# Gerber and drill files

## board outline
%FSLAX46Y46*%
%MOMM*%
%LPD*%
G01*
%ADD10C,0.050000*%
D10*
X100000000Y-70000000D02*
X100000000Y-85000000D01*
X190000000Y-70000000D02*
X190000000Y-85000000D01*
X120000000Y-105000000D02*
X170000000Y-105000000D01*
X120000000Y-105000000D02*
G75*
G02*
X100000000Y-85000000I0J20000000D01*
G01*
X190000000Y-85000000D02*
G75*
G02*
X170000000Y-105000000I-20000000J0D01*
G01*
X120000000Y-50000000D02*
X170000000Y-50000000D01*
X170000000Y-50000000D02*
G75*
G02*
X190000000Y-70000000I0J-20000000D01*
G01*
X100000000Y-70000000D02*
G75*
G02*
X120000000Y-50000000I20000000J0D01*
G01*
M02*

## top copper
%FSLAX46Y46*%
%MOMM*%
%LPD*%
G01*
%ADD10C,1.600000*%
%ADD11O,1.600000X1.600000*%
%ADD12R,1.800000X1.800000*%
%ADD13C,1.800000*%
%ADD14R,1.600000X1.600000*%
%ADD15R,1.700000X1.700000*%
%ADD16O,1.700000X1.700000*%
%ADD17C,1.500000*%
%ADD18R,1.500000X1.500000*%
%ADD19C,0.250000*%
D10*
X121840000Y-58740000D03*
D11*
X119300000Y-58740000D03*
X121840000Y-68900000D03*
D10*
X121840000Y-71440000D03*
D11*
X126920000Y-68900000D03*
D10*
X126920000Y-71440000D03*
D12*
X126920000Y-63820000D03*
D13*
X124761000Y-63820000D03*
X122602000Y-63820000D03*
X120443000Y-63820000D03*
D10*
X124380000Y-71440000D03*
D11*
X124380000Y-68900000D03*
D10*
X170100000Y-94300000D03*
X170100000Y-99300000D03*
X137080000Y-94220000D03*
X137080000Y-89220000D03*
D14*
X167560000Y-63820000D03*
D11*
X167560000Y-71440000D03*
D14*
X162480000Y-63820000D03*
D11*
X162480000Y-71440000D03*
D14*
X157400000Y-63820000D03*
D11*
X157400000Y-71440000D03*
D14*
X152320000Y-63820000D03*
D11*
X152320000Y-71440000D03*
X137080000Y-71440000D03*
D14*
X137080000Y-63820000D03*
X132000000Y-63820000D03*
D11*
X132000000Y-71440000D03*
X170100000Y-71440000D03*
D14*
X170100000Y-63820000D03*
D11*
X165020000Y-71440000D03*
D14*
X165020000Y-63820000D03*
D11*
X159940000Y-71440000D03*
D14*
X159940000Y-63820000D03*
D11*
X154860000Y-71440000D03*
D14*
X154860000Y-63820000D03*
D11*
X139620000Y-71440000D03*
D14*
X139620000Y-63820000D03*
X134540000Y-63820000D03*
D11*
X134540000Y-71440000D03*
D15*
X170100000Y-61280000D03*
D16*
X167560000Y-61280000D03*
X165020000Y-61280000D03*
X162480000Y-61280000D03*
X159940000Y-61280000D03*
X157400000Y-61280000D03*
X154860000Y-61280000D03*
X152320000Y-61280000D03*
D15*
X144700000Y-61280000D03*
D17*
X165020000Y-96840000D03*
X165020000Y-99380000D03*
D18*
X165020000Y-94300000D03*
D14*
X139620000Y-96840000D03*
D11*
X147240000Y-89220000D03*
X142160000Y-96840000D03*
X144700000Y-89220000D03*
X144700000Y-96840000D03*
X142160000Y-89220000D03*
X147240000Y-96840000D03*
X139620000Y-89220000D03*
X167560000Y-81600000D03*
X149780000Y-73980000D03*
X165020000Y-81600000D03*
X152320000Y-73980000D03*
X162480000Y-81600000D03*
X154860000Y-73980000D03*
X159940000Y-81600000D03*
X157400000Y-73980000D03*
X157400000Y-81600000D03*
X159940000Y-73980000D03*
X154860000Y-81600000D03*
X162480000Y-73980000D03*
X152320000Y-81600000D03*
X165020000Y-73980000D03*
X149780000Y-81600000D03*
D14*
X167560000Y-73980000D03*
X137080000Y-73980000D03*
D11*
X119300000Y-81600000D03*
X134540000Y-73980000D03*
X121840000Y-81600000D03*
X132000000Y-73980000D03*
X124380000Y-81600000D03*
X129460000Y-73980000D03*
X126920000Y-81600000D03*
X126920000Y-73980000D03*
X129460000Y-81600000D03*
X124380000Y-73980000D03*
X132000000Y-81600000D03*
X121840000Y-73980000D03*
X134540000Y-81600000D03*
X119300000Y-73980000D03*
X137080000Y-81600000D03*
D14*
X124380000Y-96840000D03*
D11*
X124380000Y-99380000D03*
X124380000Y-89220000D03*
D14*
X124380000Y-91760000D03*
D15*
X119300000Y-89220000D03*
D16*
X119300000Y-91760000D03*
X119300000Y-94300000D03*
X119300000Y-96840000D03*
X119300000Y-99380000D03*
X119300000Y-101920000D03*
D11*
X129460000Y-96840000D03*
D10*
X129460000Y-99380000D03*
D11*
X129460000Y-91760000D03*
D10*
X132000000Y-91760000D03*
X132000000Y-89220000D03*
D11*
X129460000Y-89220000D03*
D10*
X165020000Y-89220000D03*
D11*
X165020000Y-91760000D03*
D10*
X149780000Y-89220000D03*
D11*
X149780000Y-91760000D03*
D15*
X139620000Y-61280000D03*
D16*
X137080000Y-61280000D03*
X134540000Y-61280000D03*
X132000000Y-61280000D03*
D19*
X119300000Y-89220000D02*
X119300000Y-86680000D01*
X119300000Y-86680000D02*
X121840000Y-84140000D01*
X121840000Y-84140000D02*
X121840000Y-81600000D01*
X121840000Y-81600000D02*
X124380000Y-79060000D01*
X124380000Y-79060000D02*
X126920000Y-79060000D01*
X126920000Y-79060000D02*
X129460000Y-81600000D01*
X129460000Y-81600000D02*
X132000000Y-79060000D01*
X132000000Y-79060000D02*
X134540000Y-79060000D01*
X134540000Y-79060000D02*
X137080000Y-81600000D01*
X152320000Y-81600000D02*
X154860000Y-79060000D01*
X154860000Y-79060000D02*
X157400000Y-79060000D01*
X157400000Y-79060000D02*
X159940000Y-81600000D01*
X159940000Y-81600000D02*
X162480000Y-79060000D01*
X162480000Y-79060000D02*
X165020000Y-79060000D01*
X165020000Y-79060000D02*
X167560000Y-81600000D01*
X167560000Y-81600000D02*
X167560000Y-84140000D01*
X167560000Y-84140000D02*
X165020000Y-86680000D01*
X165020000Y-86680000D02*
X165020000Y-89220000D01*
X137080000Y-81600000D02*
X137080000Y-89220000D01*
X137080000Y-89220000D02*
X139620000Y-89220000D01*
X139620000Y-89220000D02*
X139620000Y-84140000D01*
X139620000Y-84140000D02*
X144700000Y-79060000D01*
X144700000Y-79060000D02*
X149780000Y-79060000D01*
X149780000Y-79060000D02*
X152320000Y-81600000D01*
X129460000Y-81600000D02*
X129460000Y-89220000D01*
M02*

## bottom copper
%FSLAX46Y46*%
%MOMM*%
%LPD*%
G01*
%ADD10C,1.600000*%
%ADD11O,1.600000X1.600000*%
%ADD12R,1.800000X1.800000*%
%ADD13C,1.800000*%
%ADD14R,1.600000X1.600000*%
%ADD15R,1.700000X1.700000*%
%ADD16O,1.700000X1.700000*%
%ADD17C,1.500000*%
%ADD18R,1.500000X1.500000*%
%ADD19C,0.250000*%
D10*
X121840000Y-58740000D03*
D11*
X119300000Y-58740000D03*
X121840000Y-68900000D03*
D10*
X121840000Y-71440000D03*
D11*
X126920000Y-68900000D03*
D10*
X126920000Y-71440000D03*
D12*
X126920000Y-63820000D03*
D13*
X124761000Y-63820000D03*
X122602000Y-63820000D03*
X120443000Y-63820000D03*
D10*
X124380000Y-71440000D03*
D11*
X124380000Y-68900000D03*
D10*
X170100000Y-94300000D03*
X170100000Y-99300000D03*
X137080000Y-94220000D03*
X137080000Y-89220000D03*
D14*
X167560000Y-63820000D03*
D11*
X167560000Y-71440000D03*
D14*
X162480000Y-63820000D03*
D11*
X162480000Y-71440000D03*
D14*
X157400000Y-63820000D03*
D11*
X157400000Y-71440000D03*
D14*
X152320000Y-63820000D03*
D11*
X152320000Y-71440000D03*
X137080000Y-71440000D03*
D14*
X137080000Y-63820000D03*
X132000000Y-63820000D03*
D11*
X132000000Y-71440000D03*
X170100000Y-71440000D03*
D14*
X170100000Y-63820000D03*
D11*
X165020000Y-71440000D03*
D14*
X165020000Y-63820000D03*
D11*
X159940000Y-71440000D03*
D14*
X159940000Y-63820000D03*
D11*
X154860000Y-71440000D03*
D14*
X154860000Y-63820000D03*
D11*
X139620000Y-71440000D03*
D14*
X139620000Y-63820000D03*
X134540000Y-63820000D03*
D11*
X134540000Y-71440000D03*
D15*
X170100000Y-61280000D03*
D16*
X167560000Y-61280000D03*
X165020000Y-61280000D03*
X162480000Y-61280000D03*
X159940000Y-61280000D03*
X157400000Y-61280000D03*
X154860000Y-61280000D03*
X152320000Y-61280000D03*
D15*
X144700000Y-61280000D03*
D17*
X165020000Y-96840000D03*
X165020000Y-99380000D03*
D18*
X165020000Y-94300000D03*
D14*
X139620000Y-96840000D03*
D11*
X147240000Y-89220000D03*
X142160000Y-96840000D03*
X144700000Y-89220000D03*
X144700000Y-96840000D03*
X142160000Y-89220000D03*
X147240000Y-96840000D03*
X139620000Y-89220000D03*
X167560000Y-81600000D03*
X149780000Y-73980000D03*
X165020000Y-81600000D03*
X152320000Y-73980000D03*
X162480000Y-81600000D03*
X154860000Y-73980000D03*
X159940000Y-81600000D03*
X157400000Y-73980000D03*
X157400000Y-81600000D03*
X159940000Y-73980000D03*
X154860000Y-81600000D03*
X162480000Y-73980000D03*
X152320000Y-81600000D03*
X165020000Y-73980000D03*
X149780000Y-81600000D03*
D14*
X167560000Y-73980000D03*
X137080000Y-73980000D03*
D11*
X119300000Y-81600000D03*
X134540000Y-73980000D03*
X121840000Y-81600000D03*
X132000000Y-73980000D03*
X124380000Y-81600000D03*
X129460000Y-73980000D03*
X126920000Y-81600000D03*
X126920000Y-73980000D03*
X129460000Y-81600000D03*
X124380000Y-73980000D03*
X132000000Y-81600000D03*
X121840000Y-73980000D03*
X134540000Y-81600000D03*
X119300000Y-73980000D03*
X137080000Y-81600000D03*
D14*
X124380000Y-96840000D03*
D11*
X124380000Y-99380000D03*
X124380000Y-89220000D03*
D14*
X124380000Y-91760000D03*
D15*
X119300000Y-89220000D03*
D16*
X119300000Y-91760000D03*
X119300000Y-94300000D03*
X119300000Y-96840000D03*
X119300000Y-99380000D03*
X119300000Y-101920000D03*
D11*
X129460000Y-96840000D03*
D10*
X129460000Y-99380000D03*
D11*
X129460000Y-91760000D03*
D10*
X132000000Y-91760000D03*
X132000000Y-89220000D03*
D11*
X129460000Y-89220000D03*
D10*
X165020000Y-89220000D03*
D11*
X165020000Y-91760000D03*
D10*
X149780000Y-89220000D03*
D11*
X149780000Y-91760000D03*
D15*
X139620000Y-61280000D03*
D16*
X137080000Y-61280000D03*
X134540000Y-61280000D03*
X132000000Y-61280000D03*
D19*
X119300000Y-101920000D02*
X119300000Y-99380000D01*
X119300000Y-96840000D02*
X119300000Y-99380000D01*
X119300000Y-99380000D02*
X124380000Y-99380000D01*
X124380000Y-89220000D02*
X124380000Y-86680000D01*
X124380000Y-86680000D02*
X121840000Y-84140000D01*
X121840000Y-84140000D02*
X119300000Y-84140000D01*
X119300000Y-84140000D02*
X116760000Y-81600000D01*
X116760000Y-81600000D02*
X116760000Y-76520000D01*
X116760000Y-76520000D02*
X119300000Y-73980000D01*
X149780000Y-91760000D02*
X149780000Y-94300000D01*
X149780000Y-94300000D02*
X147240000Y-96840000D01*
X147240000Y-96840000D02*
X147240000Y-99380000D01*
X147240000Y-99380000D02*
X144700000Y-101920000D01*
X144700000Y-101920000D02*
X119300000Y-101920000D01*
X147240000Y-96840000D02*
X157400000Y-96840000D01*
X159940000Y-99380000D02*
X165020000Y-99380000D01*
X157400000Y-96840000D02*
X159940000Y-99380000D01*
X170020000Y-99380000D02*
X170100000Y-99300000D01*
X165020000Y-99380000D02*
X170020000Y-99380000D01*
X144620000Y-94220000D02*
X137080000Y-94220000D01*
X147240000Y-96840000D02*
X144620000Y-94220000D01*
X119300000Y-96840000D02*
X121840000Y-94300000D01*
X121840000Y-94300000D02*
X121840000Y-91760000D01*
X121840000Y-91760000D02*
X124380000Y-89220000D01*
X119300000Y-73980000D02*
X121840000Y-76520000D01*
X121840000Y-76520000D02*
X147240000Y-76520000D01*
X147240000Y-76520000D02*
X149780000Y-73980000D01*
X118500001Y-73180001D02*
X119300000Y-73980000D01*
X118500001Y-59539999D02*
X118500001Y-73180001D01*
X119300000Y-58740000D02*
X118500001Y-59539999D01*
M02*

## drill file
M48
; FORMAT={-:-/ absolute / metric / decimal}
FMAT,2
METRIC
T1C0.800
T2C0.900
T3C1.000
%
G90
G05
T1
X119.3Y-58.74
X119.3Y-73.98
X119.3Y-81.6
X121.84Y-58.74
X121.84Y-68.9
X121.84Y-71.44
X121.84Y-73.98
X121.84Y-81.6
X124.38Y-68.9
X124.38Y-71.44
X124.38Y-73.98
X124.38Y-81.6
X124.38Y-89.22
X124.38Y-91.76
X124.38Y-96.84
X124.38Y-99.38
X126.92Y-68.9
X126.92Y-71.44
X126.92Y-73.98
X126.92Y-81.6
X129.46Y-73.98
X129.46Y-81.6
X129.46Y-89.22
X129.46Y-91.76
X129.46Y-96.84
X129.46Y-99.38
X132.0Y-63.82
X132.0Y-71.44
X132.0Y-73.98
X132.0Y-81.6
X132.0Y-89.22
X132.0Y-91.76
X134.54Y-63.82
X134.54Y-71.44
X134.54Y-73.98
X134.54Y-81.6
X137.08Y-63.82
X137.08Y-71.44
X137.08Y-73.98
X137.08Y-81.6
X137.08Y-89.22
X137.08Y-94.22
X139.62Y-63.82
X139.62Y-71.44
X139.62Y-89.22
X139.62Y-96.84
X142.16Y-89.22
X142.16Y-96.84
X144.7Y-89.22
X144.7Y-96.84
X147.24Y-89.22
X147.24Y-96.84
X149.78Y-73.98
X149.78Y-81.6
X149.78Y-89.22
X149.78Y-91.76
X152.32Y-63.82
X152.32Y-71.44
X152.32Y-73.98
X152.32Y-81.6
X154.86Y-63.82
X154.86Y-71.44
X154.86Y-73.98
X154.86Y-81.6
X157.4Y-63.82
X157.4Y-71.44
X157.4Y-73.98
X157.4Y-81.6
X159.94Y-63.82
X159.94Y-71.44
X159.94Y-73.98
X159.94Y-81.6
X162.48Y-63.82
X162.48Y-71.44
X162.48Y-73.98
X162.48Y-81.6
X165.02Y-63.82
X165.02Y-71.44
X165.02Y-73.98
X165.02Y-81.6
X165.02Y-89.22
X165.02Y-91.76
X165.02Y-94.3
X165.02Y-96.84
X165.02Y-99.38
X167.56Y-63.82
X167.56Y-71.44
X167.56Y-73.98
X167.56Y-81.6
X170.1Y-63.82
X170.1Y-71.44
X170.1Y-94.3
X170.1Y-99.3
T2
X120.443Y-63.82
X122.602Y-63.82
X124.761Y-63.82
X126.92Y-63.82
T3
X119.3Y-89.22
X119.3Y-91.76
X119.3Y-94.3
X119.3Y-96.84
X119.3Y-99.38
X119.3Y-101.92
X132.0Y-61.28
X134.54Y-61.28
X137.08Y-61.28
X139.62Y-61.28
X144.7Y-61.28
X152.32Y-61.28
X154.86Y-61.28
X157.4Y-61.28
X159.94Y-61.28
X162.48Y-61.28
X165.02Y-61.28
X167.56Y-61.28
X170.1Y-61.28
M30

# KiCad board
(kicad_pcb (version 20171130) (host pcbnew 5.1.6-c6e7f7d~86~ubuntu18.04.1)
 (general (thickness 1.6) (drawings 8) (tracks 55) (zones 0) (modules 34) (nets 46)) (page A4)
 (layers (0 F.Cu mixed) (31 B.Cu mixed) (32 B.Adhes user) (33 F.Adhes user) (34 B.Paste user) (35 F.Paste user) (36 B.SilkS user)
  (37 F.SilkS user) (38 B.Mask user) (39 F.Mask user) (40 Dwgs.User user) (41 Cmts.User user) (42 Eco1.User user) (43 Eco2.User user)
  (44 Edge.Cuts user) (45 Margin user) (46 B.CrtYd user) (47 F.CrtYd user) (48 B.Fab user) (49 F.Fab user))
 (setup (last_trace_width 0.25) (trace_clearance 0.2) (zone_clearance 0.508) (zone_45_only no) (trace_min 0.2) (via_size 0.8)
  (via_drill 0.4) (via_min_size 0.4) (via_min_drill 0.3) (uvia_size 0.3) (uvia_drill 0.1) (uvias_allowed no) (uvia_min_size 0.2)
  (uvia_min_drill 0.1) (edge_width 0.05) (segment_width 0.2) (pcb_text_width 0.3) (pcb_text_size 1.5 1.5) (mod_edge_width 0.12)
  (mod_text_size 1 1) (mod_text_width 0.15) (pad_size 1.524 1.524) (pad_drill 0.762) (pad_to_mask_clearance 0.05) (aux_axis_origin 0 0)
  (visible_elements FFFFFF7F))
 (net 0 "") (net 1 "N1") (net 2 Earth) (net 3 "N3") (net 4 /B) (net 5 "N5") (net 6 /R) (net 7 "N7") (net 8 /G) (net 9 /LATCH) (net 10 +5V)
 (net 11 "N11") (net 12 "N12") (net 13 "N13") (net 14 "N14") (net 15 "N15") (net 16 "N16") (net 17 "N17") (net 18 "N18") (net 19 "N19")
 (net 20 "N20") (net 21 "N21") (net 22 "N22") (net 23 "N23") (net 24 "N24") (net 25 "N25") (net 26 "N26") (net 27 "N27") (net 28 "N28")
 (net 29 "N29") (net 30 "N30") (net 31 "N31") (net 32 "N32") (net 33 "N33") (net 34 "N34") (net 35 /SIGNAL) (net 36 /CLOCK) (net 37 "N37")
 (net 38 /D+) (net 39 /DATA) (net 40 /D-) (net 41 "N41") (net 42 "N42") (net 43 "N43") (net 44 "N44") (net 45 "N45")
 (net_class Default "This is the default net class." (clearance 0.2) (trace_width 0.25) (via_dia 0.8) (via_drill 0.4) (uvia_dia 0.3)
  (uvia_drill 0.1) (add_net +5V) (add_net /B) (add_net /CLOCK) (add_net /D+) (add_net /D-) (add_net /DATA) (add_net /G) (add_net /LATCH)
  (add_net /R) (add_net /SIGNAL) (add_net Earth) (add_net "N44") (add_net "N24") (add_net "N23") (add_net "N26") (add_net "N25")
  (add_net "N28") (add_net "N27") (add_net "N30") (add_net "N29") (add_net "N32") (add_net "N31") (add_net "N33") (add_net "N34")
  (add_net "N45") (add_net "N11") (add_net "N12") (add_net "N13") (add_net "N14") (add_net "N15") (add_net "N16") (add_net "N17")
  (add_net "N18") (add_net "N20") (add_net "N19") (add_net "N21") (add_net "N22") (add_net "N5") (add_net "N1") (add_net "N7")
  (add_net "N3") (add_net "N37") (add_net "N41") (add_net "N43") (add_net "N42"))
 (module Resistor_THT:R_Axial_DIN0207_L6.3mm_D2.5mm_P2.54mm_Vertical (layer F.Cu) (at 121.84 58.74 180)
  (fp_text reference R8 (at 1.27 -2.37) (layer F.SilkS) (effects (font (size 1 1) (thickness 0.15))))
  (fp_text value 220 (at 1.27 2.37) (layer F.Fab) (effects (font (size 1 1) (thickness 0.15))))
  (pad 1 thru_hole circle (at 0 0 180) (size 1.6 1.6) (drill 0.8) (layers *.Cu *.Mask) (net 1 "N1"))
  (pad 2 thru_hole oval (at 2.54 0 180) (size 1.6 1.6) (drill 0.8) (layers *.Cu *.Mask) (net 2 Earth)))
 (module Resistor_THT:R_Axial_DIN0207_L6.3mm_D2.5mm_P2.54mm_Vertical (layer F.Cu) (at 121.84 71.44 90)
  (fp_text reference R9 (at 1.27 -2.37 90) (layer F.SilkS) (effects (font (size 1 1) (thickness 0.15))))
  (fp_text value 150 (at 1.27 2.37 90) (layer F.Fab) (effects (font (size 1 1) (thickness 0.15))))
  (pad 2 thru_hole oval (at 2.54 0 90) (size 1.6 1.6) (drill 0.8) (layers *.Cu *.Mask) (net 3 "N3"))
  (pad 1 thru_hole circle (at 0 0 90) (size 1.6 1.6) (drill 0.8) (layers *.Cu *.Mask) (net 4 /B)))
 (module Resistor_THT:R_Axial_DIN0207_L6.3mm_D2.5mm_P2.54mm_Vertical (layer F.Cu) (at 126.92 71.44 90)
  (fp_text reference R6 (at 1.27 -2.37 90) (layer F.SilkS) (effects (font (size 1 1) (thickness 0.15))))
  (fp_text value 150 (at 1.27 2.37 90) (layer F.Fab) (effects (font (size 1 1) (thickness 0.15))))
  (pad 2 thru_hole oval (at 2.54 0 90) (size 1.6 1.6) (drill 0.8) (layers *.Cu *.Mask) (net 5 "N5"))
  (pad 1 thru_hole circle (at 0 0 90) (size 1.6 1.6) (drill 0.8) (layers *.Cu *.Mask) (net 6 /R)))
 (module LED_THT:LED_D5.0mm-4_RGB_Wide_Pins (layer F.Cu) (at 126.92 63.82 180)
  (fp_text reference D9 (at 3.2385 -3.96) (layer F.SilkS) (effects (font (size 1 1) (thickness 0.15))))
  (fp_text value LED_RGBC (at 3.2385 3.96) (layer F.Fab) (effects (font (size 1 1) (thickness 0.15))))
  (pad 1 thru_hole rect (at 0 0 180) (size 1.8 1.8) (drill 0.9) (layers *.Cu *.Mask) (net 5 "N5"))
  (pad 2 thru_hole circle (at 2.159 0 180) (size 1.8 1.8) (drill 0.9) (layers *.Cu *.Mask) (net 1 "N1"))
  (pad 3 thru_hole circle (at 4.318 0 180) (size 1.8 1.8) (drill 0.9) (layers *.Cu *.Mask) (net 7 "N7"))
  (pad 4 thru_hole circle (at 6.477 0 180) (size 1.8 1.8) (drill 0.9) (layers *.Cu *.Mask) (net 3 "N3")))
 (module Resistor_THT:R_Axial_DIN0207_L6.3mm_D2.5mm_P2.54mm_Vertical (layer F.Cu) (at 124.38 71.44 90)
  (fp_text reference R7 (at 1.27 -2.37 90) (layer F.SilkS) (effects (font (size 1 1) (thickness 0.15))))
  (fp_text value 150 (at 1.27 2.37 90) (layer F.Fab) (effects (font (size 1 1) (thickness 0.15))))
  (pad 1 thru_hole circle (at 0 0 90) (size 1.6 1.6) (drill 0.8) (layers *.Cu *.Mask) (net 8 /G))
  (pad 2 thru_hole oval (at 2.54 0 90) (size 1.6 1.6) (drill 0.8) (layers *.Cu *.Mask) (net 7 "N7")))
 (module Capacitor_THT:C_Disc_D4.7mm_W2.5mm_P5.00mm (layer F.Cu) (at 170.1 94.3 270)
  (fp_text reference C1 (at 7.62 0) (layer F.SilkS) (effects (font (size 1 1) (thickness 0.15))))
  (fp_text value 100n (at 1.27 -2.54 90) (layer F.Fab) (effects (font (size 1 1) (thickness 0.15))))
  (pad 1 thru_hole circle (at 0 0 270) (size 1.6 1.6) (drill 0.8) (layers *.Cu *.Mask) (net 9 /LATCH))
  (pad 2 thru_hole circle (at 5 0 270) (size 1.6 1.6) (drill 0.8) (layers *.Cu *.Mask) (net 2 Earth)))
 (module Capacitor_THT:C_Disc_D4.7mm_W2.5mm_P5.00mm (layer F.Cu) (at 137.08 89.22 270)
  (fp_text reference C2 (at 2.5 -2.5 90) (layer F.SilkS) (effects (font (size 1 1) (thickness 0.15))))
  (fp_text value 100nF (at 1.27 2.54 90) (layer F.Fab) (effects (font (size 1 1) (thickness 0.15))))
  (pad 2 thru_hole circle (at 5 0 270) (size 1.6 1.6) (drill 0.8) (layers *.Cu *.Mask) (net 2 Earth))
  (pad 1 thru_hole circle (at 0 0 270) (size 1.6 1.6) (drill 0.8) (layers *.Cu *.Mask) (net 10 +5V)))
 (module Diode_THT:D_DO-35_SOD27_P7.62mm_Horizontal (layer F.Cu) (at 167.56 63.82 270)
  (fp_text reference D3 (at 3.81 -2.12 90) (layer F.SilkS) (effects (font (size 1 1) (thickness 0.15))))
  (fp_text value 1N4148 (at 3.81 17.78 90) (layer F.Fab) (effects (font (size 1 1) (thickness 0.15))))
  (pad 1 thru_hole rect (at 0 0 270) (size 1.6 1.6) (drill 0.8) (layers *.Cu *.Mask) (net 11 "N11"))
  (pad 2 thru_hole oval (at 7.62 0 270) (size 1.6 1.6) (drill 0.8) (layers *.Cu *.Mask) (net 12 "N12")))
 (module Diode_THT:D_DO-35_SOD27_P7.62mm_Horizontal (layer F.Cu) (at 162.48 63.82 270)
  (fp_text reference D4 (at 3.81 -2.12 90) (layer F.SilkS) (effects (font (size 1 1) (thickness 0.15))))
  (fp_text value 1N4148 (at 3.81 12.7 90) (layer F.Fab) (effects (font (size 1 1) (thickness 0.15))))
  (pad 1 thru_hole rect (at 0 0 270) (size 1.6 1.6) (drill 0.8) (layers *.Cu *.Mask) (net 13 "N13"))
  (pad 2 thru_hole oval (at 7.62 0 270) (size 1.6 1.6) (drill 0.8) (layers *.Cu *.Mask) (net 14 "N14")))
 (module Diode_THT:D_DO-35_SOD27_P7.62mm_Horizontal (layer F.Cu) (at 157.4 63.82 270)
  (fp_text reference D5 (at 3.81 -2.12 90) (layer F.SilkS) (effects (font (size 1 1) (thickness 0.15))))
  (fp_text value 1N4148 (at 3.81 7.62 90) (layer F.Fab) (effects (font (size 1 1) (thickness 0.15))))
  (pad 1 thru_hole rect (at 0 0 270) (size 1.6 1.6) (drill 0.8) (layers *.Cu *.Mask) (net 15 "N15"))
  (pad 2 thru_hole oval (at 7.62 0 270) (size 1.6 1.6) (drill 0.8) (layers *.Cu *.Mask) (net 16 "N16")))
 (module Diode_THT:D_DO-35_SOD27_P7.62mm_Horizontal (layer F.Cu) (at 152.32 63.82 270)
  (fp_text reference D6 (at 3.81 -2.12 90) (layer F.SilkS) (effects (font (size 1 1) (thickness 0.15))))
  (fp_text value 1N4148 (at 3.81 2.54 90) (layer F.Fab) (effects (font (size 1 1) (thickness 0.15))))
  (pad 1 thru_hole rect (at 0 0 270) (size 1.6 1.6) (drill 0.8) (layers *.Cu *.Mask) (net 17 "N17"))
  (pad 2 thru_hole oval (at 7.62 0 270) (size 1.6 1.6) (drill 0.8) (layers *.Cu *.Mask) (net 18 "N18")))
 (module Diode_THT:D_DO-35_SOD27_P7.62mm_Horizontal (layer F.Cu) (at 137.08 63.82 270)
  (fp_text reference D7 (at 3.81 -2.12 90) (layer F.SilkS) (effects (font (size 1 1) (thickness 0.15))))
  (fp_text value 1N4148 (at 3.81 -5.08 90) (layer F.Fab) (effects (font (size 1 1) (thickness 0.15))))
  (pad 2 thru_hole oval (at 7.62 0 270) (size 1.6 1.6) (drill 0.8) (layers *.Cu *.Mask) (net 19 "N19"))
  (pad 1 thru_hole rect (at 0 0 270) (size 1.6 1.6) (drill 0.8) (layers *.Cu *.Mask) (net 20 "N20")))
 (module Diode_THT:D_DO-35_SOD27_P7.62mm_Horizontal (layer F.Cu) (at 132 63.82 270)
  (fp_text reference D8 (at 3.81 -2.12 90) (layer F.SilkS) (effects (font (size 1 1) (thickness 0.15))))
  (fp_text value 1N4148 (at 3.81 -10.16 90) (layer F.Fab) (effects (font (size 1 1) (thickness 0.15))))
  (pad 1 thru_hole rect (at 0 0 270) (size 1.6 1.6) (drill 0.8) (layers *.Cu *.Mask) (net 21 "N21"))
  (pad 2 thru_hole oval (at 7.62 0 270) (size 1.6 1.6) (drill 0.8) (layers *.Cu *.Mask) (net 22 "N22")))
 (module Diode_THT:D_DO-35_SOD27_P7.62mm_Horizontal (layer F.Cu) (at 170.1 63.82 270)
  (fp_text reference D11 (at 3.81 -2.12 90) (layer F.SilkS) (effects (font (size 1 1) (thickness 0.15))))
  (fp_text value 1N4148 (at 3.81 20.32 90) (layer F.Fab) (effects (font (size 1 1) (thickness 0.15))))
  (pad 2 thru_hole oval (at 7.62 0 270) (size 1.6 1.6) (drill 0.8) (layers *.Cu *.Mask) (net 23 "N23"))
  (pad 1 thru_hole rect (at 0 0 270) (size 1.6 1.6) (drill 0.8) (layers *.Cu *.Mask) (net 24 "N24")))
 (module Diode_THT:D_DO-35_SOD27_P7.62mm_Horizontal (layer F.Cu) (at 165.02 63.82 270)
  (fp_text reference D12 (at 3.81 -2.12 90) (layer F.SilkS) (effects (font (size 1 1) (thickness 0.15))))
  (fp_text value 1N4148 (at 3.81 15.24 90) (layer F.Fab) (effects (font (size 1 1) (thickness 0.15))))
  (pad 2 thru_hole oval (at 7.62 0 270) (size 1.6 1.6) (drill 0.8) (layers *.Cu *.Mask) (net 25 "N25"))
  (pad 1 thru_hole rect (at 0 0 270) (size 1.6 1.6) (drill 0.8) (layers *.Cu *.Mask) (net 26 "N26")))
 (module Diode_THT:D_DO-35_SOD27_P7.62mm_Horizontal (layer F.Cu) (at 159.94 63.82 270)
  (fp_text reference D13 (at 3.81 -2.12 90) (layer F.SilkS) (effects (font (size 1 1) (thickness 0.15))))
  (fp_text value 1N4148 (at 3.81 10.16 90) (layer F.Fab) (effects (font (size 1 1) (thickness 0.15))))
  (pad 2 thru_hole oval (at 7.62 0 270) (size 1.6 1.6) (drill 0.8) (layers *.Cu *.Mask) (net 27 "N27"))
  (pad 1 thru_hole rect (at 0 0 270) (size 1.6 1.6) (drill 0.8) (layers *.Cu *.Mask) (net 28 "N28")))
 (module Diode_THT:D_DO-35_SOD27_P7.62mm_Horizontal (layer F.Cu) (at 154.86 63.82 270)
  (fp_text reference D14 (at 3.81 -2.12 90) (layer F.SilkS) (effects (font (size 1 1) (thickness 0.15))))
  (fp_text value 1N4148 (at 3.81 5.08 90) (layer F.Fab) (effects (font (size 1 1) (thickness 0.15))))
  (pad 2 thru_hole oval (at 7.62 0 270) (size 1.6 1.6) (drill 0.8) (layers *.Cu *.Mask) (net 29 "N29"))
  (pad 1 thru_hole rect (at 0 0 270) (size 1.6 1.6) (drill 0.8) (layers *.Cu *.Mask) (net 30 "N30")))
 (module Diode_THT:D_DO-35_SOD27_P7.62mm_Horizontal (layer F.Cu) (at 139.62 63.82 270)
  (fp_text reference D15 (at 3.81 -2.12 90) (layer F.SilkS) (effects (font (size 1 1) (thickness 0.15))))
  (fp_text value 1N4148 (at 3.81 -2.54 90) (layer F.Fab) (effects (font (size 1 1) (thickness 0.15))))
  (pad 2 thru_hole oval (at 7.62 0 270) (size 1.6 1.6) (drill 0.8) (layers *.Cu *.Mask) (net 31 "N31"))
  (pad 1 thru_hole rect (at 0 0 270) (size 1.6 1.6) (drill 0.8) (layers *.Cu *.Mask) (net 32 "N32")))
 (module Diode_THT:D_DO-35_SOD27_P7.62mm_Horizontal (layer F.Cu) (at 134.54 63.82 270)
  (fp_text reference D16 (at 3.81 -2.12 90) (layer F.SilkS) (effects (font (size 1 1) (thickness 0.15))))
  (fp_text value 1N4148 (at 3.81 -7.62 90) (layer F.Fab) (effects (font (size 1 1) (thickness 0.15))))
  (pad 1 thru_hole rect (at 0 0 270) (size 1.6 1.6) (drill 0.8) (layers *.Cu *.Mask) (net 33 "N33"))
  (pad 2 thru_hole oval (at 7.62 0 270) (size 1.6 1.6) (drill 0.8) (layers *.Cu *.Mask) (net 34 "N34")))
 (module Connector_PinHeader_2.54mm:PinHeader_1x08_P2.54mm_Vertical (layer F.Cu) (at 170.1 61.28 270)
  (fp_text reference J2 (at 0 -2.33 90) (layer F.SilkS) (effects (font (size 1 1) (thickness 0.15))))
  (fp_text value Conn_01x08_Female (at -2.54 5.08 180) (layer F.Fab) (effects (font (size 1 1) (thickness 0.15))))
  (pad 1 thru_hole rect (at 0 0 270) (size 1.7 1.7) (drill 1) (layers *.Cu *.Mask) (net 24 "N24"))
  (pad 2 thru_hole oval (at 0 2.54 270) (size 1.7 1.7) (drill 1) (layers *.Cu *.Mask) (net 11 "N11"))
  (pad 3 thru_hole oval (at 0 5.08 270) (size 1.7 1.7) (drill 1) (layers *.Cu *.Mask) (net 26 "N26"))
  (pad 4 thru_hole oval (at 0 7.62 270) (size 1.7 1.7) (drill 1) (layers *.Cu *.Mask) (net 13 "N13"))
  (pad 5 thru_hole oval (at 0 10.16 270) (size 1.7 1.7) (drill 1) (layers *.Cu *.Mask) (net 28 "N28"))
  (pad 6 thru_hole oval (at 0 12.7 270) (size 1.7 1.7) (drill 1) (layers *.Cu *.Mask) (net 15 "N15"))
  (pad 7 thru_hole oval (at 0 15.24 270) (size 1.7 1.7) (drill 1) (layers *.Cu *.Mask) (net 30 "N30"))
  (pad 8 thru_hole oval (at 0 17.78 270) (size 1.7 1.7) (drill 1) (layers *.Cu *.Mask) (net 17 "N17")))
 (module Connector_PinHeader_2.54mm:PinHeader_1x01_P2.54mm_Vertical (layer F.Cu) (at 144.7 61.28)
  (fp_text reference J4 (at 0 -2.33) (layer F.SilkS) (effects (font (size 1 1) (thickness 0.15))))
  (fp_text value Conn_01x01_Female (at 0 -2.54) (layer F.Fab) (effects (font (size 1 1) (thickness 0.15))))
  (pad 1 thru_hole rect (at 0 0) (size 1.7 1.7) (drill 1) (layers *.Cu *.Mask) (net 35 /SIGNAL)))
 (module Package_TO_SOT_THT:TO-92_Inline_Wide (layer F.Cu) (at 165.02 94.3 270)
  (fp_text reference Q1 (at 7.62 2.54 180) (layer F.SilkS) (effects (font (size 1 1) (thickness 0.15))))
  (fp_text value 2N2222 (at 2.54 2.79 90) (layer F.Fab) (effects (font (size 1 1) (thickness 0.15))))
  (pad 2 thru_hole circle (at 2.54 0) (size 1.5 1.5) (drill 0.8) (layers *.Cu *.Mask) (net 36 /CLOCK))
  (pad 3 thru_hole circle (at 5.08 0) (size 1.5 1.5) (drill 0.8) (layers *.Cu *.Mask) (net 2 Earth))
  (pad 1 thru_hole rect (at 0 0) (size 1.5 1.5) (drill 0.8) (layers *.Cu *.Mask) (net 9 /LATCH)))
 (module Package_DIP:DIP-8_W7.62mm (layer F.Cu) (at 139.62 96.84 90)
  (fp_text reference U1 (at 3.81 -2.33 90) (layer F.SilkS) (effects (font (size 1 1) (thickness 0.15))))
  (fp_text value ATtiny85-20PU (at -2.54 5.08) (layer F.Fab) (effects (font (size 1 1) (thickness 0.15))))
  (pad 1 thru_hole rect (at 0 0 90) (size 1.6 1.6) (drill 0.8) (layers *.Cu *.Mask) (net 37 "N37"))
  (pad 5 thru_hole oval (at 7.62 7.62 90) (size 1.6 1.6) (drill 0.8) (layers *.Cu *.Mask) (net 35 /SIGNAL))
  (pad 2 thru_hole oval (at 0 2.54 90) (size 1.6 1.6) (drill 0.8) (layers *.Cu *.Mask) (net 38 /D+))
  (pad 6 thru_hole oval (at 7.62 5.08 90) (size 1.6 1.6) (drill 0.8) (layers *.Cu *.Mask) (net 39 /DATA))
  (pad 3 thru_hole oval (at 0 5.08 90) (size 1.6 1.6) (drill 0.8) (layers *.Cu *.Mask) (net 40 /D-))
  (pad 7 thru_hole oval (at 7.62 2.54 90) (size 1.6 1.6) (drill 0.8) (layers *.Cu *.Mask) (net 36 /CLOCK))
  (pad 4 thru_hole oval (at 0 7.62 90) (size 1.6 1.6) (drill 0.8) (layers *.Cu *.Mask) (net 2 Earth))
  (pad 8 thru_hole oval (at 7.62 0 90) (size 1.6 1.6) (drill 0.8) (layers *.Cu *.Mask) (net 10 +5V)))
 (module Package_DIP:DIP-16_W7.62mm (layer F.Cu) (at 167.56 73.98 270)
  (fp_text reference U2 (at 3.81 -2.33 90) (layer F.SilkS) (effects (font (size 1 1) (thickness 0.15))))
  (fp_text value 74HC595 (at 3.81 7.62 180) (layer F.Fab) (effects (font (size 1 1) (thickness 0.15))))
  (pad 16 thru_hole oval (at 7.62 0 270) (size 1.6 1.6) (drill 0.8) (layers *.Cu *.Mask) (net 10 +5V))
  (pad 8 thru_hole oval (at 0 17.78 270) (size 1.6 1.6) (drill 0.8) (layers *.Cu *.Mask) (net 2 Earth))
  (pad 15 thru_hole oval (at 7.62 2.54 270) (size 1.6 1.6) (drill 0.8) (layers *.Cu *.Mask) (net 23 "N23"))
  (pad 7 thru_hole oval (at 0 15.24 270) (size 1.6 1.6) (drill 0.8) (layers *.Cu *.Mask) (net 18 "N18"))
  (pad 14 thru_hole oval (at 7.62 5.08 270) (size 1.6 1.6) (drill 0.8) (layers *.Cu *.Mask) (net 39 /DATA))
  (pad 6 thru_hole oval (at 0 12.7 270) (size 1.6 1.6) (drill 0.8) (layers *.Cu *.Mask) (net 29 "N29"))
  (pad 13 thru_hole oval (at 7.62 7.62 270) (size 1.6 1.6) (drill 0.8) (layers *.Cu *.Mask) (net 10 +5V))
  (pad 5 thru_hole oval (at 0 10.16 270) (size 1.6 1.6) (drill 0.8) (layers *.Cu *.Mask) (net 16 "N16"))
  (pad 12 thru_hole oval (at 7.62 10.16 270) (size 1.6 1.6) (drill 0.8) (layers *.Cu *.Mask) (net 9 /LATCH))
  (pad 4 thru_hole oval (at 0 7.62 270) (size 1.6 1.6) (drill 0.8) (layers *.Cu *.Mask) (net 27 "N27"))
  (pad 11 thru_hole oval (at 7.62 12.7 270) (size 1.6 1.6) (drill 0.8) (layers *.Cu *.Mask) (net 36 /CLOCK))
  (pad 3 thru_hole oval (at 0 5.08 270) (size 1.6 1.6) (drill 0.8) (layers *.Cu *.Mask) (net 14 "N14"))
  (pad 10 thru_hole oval (at 7.62 15.24 270) (size 1.6 1.6) (drill 0.8) (layers *.Cu *.Mask) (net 10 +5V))
  (pad 2 thru_hole oval (at 0 2.54 270) (size 1.6 1.6) (drill 0.8) (layers *.Cu *.Mask) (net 25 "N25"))
  (pad 9 thru_hole oval (at 7.62 17.78 270) (size 1.6 1.6) (drill 0.8) (layers *.Cu *.Mask) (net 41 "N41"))
  (pad 1 thru_hole rect (at 0 0 270) (size 1.6 1.6) (drill 0.8) (layers *.Cu *.Mask) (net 12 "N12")))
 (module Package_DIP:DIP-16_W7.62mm (layer F.Cu) (at 137.08 73.98 270)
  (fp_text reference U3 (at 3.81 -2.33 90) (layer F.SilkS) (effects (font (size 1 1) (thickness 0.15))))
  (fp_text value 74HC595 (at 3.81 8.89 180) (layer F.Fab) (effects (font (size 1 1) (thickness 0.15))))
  (pad 1 thru_hole rect (at 0 0 270) (size 1.6 1.6) (drill 0.8) (layers *.Cu *.Mask) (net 19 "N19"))
  (pad 9 thru_hole oval (at 7.62 17.78 270) (size 1.6 1.6) (drill 0.8) (layers *.Cu *.Mask) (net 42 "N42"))
  (pad 2 thru_hole oval (at 0 2.54 270) (size 1.6 1.6) (drill 0.8) (layers *.Cu *.Mask) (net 34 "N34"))
  (pad 10 thru_hole oval (at 7.62 15.24 270) (size 1.6 1.6) (drill 0.8) (layers *.Cu *.Mask) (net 10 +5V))
  (pad 3 thru_hole oval (at 0 5.08 270) (size 1.6 1.6) (drill 0.8) (layers *.Cu *.Mask) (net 22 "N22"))
  (pad 11 thru_hole oval (at 7.62 12.7 270) (size 1.6 1.6) (drill 0.8) (layers *.Cu *.Mask) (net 36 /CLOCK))
  (pad 4 thru_hole oval (at 0 7.62 270) (size 1.6 1.6) (drill 0.8) (layers *.Cu *.Mask) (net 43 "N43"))
  (pad 12 thru_hole oval (at 7.62 10.16 270) (size 1.6 1.6) (drill 0.8) (layers *.Cu *.Mask) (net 9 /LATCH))
  (pad 5 thru_hole oval (at 0 10.16 270) (size 1.6 1.6) (drill 0.8) (layers *.Cu *.Mask) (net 6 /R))
  (pad 13 thru_hole oval (at 7.62 7.62 270) (size 1.6 1.6) (drill 0.8) (layers *.Cu *.Mask) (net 10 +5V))
  (pad 6 thru_hole oval (at 0 12.7 270) (size 1.6 1.6) (drill 0.8) (layers *.Cu *.Mask) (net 8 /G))
  (pad 14 thru_hole oval (at 7.62 5.08 270) (size 1.6 1.6) (drill 0.8) (layers *.Cu *.Mask) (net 41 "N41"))
  (pad 7 thru_hole oval (at 0 15.24 270) (size 1.6 1.6) (drill 0.8) (layers *.Cu *.Mask) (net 4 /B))
  (pad 15 thru_hole oval (at 7.62 2.54 270) (size 1.6 1.6) (drill 0.8) (layers *.Cu *.Mask) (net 31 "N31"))
  (pad 8 thru_hole oval (at 0 17.78 270) (size 1.6 1.6) (drill 0.8) (layers *.Cu *.Mask) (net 2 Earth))
  (pad 16 thru_hole oval (at 7.62 0 270) (size 1.6 1.6) (drill 0.8) (layers *.Cu *.Mask) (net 10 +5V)))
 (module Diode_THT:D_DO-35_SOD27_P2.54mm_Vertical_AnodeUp (layer F.Cu) (at 124.38 96.84 270)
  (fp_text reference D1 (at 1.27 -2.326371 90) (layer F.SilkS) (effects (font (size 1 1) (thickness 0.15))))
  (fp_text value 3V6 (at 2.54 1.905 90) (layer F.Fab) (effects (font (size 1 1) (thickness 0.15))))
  (pad 1 thru_hole rect (at 0 0 270) (size 1.6 1.6) (drill 0.8) (layers *.Cu *.Mask) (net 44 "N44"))
  (pad 2 thru_hole oval (at 2.54 0 270) (size 1.6 1.6) (drill 0.8) (layers *.Cu *.Mask) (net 2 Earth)))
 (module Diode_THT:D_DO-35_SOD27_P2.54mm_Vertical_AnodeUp (layer F.Cu) (at 124.38 91.76 90)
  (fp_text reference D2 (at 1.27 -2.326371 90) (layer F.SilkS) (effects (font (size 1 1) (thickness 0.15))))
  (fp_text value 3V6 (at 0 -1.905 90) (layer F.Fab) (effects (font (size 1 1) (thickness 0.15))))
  (pad 2 thru_hole oval (at 2.54 0 90) (size 1.6 1.6) (drill 0.8) (layers *.Cu *.Mask) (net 2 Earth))
  (pad 1 thru_hole rect (at 0 0 90) (size 1.6 1.6) (drill 0.8) (layers *.Cu *.Mask) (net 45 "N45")))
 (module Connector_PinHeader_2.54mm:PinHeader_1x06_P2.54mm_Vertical (layer F.Cu) (at 119.3 89.22)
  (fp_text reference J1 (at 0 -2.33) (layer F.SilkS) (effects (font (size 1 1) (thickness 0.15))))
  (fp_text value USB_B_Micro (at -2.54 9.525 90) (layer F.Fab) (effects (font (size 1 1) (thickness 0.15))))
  (pad 1 thru_hole rect (at 0 0) (size 1.7 1.7) (drill 1) (layers *.Cu *.Mask) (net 10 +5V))
  (pad 2 thru_hole oval (at 0 2.54) (size 1.7 1.7) (drill 1) (layers *.Cu *.Mask) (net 45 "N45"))
  (pad 3 thru_hole oval (at 0 5.08) (size 1.7 1.7) (drill 1) (layers *.Cu *.Mask) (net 44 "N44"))
  (pad 4 thru_hole oval (at 0 7.62) (size 1.7 1.7) (drill 1) (layers *.Cu *.Mask) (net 2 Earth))
  (pad 5 thru_hole oval (at 0 10.16) (size 1.7 1.7) (drill 1) (layers *.Cu *.Mask) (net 2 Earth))
  (pad 6 thru_hole oval (at 0 12.7) (size 1.7 1.7) (drill 1) (layers *.Cu *.Mask) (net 2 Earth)))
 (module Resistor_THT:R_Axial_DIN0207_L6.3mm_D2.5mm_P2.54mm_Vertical (layer F.Cu) (at 129.46 99.38 90)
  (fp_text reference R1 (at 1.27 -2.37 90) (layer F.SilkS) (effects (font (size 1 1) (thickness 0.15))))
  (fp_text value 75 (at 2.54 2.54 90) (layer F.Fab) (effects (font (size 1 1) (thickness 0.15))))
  (pad 2 thru_hole oval (at 2.54 0 90) (size 1.6 1.6) (drill 0.8) (layers *.Cu *.Mask) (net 44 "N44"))
  (pad 1 thru_hole circle (at 0 0 90) (size 1.6 1.6) (drill 0.8) (layers *.Cu *.Mask) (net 38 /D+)))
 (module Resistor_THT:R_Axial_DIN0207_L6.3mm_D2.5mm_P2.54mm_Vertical (layer F.Cu) (at 132 91.76 180)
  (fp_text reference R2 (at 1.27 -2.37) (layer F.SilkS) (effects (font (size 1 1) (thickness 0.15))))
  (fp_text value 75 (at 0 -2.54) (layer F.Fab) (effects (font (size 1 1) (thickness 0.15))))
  (pad 2 thru_hole oval (at 2.54 0 180) (size 1.6 1.6) (drill 0.8) (layers *.Cu *.Mask) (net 45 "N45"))
  (pad 1 thru_hole circle (at 0 0 180) (size 1.6 1.6) (drill 0.8) (layers *.Cu *.Mask) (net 40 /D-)))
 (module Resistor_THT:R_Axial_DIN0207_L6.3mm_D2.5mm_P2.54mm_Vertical (layer F.Cu) (at 132 89.22 180)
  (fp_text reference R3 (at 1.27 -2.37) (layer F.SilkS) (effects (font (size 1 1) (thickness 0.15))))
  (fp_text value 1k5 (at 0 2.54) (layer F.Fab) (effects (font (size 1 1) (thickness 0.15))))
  (pad 1 thru_hole circle (at 0 0 180) (size 1.6 1.6) (drill 0.8) (layers *.Cu *.Mask) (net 40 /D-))
  (pad 2 thru_hole oval (at 2.54 0 180) (size 1.6 1.6) (drill 0.8) (layers *.Cu *.Mask) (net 10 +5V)))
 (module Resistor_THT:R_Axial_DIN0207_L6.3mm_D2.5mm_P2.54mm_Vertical (layer F.Cu) (at 165.02 89.22 270)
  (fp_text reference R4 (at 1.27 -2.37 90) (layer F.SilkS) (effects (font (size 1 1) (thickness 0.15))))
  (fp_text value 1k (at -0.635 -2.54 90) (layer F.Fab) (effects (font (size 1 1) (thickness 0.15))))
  (pad 1 thru_hole circle (at 0 0 270) (size 1.6 1.6) (drill 0.8) (layers *.Cu *.Mask) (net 10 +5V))
  (pad 2 thru_hole oval (at 2.54 0 270) (size 1.6 1.6) (drill 0.8) (layers *.Cu *.Mask) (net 9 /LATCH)))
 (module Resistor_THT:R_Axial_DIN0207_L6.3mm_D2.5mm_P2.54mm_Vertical (layer F.Cu) (at 149.78 89.22 270)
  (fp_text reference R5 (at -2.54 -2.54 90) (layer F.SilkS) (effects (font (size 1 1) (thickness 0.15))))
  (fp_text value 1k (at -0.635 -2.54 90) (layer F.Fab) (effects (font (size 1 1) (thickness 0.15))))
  (pad 1 thru_hole circle (at 0 0 270) (size 1.6 1.6) (drill 0.8) (layers *.Cu *.Mask) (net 35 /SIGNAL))
  (pad 2 thru_hole oval (at 2.54 0 270) (size 1.6 1.6) (drill 0.8) (layers *.Cu *.Mask) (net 2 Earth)))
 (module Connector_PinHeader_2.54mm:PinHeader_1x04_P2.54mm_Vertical (layer F.Cu) (at 139.62 61.28 270)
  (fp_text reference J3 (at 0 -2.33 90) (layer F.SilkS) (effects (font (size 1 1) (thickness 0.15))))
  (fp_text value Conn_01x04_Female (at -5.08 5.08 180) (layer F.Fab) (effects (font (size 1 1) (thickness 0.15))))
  (pad 1 thru_hole rect (at 0 0 270) (size 1.7 1.7) (drill 1) (layers *.Cu *.Mask) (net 32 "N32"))
  (pad 2 thru_hole oval (at 0 2.54 270) (size 1.7 1.7) (drill 1) (layers *.Cu *.Mask) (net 20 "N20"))
  (pad 3 thru_hole oval (at 0 5.08 270) (size 1.7 1.7) (drill 1) (layers *.Cu *.Mask) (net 33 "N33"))
  (pad 4 thru_hole oval (at 0 7.62 270) (size 1.7 1.7) (drill 1) (layers *.Cu *.Mask) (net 21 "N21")))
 (gr_line (start 100 70) (end 100 85) (layer Edge.Cuts) (width 0.05))
 (gr_line (start 190 70) (end 190 85) (layer Edge.Cuts) (width 0.05))
 (gr_line (start 120 105) (end 170 105) (layer Edge.Cuts) (width 0.05))
 (gr_arc (start 120 85) (end 100 85) (angle -90) (layer Edge.Cuts) (width 0.05))
 (gr_arc (start 170 85) (end 170 105) (angle -90) (layer Edge.Cuts) (width 0.05))
 (gr_line (start 120 50) (end 170 50) (layer Edge.Cuts) (width 0.05))
 (gr_arc (start 170 70) (end 190 70) (angle -90) (layer Edge.Cuts) (width 0.05))
 (gr_arc (start 120 70) (end 120 50) (angle -90) (layer Edge.Cuts) (width 0.05))
 (segment (start 119.3 101.92) (end 119.3 99.38) (width 0.25) (layer B.Cu) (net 2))
 (segment (start 119.3 96.84) (end 119.3 99.38) (width 0.25) (layer B.Cu) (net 2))
 (segment (start 119.3 99.38) (end 124.38 99.38) (width 0.25) (layer B.Cu) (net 2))
 (segment (start 124.38 89.22) (end 124.38 86.68) (width 0.25) (layer B.Cu) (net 2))
 (segment (start 124.38 86.68) (end 121.84 84.14) (width 0.25) (layer B.Cu) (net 2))
 (segment (start 121.84 84.14) (end 119.3 84.14) (width 0.25) (layer B.Cu) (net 2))
 (segment (start 119.3 84.14) (end 116.76 81.6) (width 0.25) (layer B.Cu) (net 2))
 (segment (start 116.76 81.6) (end 116.76 76.52) (width 0.25) (layer B.Cu) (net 2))
 (segment (start 116.76 76.52) (end 119.3 73.98) (width 0.25) (layer B.Cu) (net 2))
 (segment (start 149.78 91.76) (end 149.78 94.3) (width 0.25) (layer B.Cu) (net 2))
 (segment (start 149.78 94.3) (end 147.24 96.84) (width 0.25) (layer B.Cu) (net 2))
 (segment (start 147.24 96.84) (end 147.24 99.38) (width 0.25) (layer B.Cu) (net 2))
 (segment (start 147.24 99.38) (end 144.7 101.92) (width 0.25) (layer B.Cu) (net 2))
 (segment (start 144.7 101.92) (end 119.3 101.92) (width 0.25) (layer B.Cu) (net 2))
 (segment (start 147.24 96.84) (end 157.4 96.84) (width 0.25) (layer B.Cu) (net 2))
 (segment (start 159.94 99.38) (end 165.02 99.38) (width 0.25) (layer B.Cu) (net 2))
 (segment (start 157.4 96.84) (end 159.94 99.38) (width 0.25) (layer B.Cu) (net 2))
 (segment (start 170.02 99.38) (end 170.1 99.3) (width 0.25) (layer B.Cu) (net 2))
 (segment (start 165.02 99.38) (end 170.02 99.38) (width 0.25) (layer B.Cu) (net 2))
 (segment (start 144.62 94.22) (end 137.08 94.22) (width 0.25) (layer B.Cu) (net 2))
 (segment (start 147.24 96.84) (end 144.62 94.22) (width 0.25) (layer B.Cu) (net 2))
 (segment (start 119.3 96.84) (end 121.84 94.3) (width 0.25) (layer B.Cu) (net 2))
 (segment (start 121.84 94.3) (end 121.84 91.76) (width 0.25) (layer B.Cu) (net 2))
 (segment (start 121.84 91.76) (end 124.38 89.22) (width 0.25) (layer B.Cu) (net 2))
 (segment (start 119.3 73.98) (end 121.84 76.52) (width 0.25) (layer B.Cu) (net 2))
 (segment (start 121.84 76.52) (end 147.24 76.52) (width 0.25) (layer B.Cu) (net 2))
 (segment (start 147.24 76.52) (end 149.78 73.98) (width 0.25) (layer B.Cu) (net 2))
 (segment (start 118.500001 73.180001) (end 119.3 73.98) (width 0.25) (layer B.Cu) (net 2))
 (segment (start 118.500001 59.539999) (end 118.500001 73.180001) (width 0.25) (layer B.Cu) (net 2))
 (segment (start 119.3 58.74) (end 118.500001 59.539999) (width 0.25) (layer B.Cu) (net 2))
 (segment (start 119.3 89.22) (end 119.3 86.68) (width 0.25) (layer F.Cu) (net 10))
 (segment (start 119.3 86.68) (end 121.84 84.14) (width 0.25) (layer F.Cu) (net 10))
 (segment (start 121.84 84.14) (end 121.84 81.6) (width 0.25) (layer F.Cu) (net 10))
 (segment (start 121.84 81.6) (end 124.38 79.06) (width 0.25) (layer F.Cu) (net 10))
 (segment (start 124.38 79.06) (end 126.92 79.06) (width 0.25) (layer F.Cu) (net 10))
 (segment (start 126.92 79.06) (end 129.46 81.6) (width 0.25) (layer F.Cu) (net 10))
 (segment (start 129.46 81.6) (end 132 79.06) (width 0.25) (layer F.Cu) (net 10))
 (segment (start 132 79.06) (end 134.54 79.06) (width 0.25) (layer F.Cu) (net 10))
 (segment (start 134.54 79.06) (end 137.08 81.6) (width 0.25) (layer F.Cu) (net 10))
 (segment (start 152.32 81.6) (end 154.86 79.06) (width 0.25) (layer F.Cu) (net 10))
 (segment (start 154.86 79.06) (end 157.4 79.06) (width 0.25) (layer F.Cu) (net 10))
 (segment (start 157.4 79.06) (end 159.94 81.6) (width 0.25) (layer F.Cu) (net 10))
 (segment (start 159.94 81.6) (end 162.48 79.06) (width 0.25) (layer F.Cu) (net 10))
 (segment (start 162.48 79.06) (end 165.02 79.06) (width 0.25) (layer F.Cu) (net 10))
 (segment (start 165.02 79.06) (end 167.56 81.6) (width 0.25) (layer F.Cu) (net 10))
 (segment (start 167.56 81.6) (end 167.56 84.14) (width 0.25) (layer F.Cu) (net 10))
 (segment (start 167.56 84.14) (end 165.02 86.68) (width 0.25) (layer F.Cu) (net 10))
 (segment (start 165.02 86.68) (end 165.02 89.22) (width 0.25) (layer F.Cu) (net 10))
 (segment (start 137.08 81.6) (end 137.08 89.22) (width 0.25) (layer F.Cu) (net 10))
 (segment (start 137.08 89.22) (end 139.62 89.22) (width 0.25) (layer F.Cu) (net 10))
 (segment (start 139.62 89.22) (end 139.62 84.14) (width 0.25) (layer F.Cu) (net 10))
 (segment (start 139.62 84.14) (end 144.7 79.06) (width 0.25) (layer F.Cu) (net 10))
 (segment (start 144.7 79.06) (end 149.78 79.06) (width 0.25) (layer F.Cu) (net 10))
 (segment (start 149.78 79.06) (end 152.32 81.6) (width 0.25) (layer F.Cu) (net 10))
 (segment (start 129.46 81.6) (end 129.46 89.22) (width 0.25) (layer F.Cu) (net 10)))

